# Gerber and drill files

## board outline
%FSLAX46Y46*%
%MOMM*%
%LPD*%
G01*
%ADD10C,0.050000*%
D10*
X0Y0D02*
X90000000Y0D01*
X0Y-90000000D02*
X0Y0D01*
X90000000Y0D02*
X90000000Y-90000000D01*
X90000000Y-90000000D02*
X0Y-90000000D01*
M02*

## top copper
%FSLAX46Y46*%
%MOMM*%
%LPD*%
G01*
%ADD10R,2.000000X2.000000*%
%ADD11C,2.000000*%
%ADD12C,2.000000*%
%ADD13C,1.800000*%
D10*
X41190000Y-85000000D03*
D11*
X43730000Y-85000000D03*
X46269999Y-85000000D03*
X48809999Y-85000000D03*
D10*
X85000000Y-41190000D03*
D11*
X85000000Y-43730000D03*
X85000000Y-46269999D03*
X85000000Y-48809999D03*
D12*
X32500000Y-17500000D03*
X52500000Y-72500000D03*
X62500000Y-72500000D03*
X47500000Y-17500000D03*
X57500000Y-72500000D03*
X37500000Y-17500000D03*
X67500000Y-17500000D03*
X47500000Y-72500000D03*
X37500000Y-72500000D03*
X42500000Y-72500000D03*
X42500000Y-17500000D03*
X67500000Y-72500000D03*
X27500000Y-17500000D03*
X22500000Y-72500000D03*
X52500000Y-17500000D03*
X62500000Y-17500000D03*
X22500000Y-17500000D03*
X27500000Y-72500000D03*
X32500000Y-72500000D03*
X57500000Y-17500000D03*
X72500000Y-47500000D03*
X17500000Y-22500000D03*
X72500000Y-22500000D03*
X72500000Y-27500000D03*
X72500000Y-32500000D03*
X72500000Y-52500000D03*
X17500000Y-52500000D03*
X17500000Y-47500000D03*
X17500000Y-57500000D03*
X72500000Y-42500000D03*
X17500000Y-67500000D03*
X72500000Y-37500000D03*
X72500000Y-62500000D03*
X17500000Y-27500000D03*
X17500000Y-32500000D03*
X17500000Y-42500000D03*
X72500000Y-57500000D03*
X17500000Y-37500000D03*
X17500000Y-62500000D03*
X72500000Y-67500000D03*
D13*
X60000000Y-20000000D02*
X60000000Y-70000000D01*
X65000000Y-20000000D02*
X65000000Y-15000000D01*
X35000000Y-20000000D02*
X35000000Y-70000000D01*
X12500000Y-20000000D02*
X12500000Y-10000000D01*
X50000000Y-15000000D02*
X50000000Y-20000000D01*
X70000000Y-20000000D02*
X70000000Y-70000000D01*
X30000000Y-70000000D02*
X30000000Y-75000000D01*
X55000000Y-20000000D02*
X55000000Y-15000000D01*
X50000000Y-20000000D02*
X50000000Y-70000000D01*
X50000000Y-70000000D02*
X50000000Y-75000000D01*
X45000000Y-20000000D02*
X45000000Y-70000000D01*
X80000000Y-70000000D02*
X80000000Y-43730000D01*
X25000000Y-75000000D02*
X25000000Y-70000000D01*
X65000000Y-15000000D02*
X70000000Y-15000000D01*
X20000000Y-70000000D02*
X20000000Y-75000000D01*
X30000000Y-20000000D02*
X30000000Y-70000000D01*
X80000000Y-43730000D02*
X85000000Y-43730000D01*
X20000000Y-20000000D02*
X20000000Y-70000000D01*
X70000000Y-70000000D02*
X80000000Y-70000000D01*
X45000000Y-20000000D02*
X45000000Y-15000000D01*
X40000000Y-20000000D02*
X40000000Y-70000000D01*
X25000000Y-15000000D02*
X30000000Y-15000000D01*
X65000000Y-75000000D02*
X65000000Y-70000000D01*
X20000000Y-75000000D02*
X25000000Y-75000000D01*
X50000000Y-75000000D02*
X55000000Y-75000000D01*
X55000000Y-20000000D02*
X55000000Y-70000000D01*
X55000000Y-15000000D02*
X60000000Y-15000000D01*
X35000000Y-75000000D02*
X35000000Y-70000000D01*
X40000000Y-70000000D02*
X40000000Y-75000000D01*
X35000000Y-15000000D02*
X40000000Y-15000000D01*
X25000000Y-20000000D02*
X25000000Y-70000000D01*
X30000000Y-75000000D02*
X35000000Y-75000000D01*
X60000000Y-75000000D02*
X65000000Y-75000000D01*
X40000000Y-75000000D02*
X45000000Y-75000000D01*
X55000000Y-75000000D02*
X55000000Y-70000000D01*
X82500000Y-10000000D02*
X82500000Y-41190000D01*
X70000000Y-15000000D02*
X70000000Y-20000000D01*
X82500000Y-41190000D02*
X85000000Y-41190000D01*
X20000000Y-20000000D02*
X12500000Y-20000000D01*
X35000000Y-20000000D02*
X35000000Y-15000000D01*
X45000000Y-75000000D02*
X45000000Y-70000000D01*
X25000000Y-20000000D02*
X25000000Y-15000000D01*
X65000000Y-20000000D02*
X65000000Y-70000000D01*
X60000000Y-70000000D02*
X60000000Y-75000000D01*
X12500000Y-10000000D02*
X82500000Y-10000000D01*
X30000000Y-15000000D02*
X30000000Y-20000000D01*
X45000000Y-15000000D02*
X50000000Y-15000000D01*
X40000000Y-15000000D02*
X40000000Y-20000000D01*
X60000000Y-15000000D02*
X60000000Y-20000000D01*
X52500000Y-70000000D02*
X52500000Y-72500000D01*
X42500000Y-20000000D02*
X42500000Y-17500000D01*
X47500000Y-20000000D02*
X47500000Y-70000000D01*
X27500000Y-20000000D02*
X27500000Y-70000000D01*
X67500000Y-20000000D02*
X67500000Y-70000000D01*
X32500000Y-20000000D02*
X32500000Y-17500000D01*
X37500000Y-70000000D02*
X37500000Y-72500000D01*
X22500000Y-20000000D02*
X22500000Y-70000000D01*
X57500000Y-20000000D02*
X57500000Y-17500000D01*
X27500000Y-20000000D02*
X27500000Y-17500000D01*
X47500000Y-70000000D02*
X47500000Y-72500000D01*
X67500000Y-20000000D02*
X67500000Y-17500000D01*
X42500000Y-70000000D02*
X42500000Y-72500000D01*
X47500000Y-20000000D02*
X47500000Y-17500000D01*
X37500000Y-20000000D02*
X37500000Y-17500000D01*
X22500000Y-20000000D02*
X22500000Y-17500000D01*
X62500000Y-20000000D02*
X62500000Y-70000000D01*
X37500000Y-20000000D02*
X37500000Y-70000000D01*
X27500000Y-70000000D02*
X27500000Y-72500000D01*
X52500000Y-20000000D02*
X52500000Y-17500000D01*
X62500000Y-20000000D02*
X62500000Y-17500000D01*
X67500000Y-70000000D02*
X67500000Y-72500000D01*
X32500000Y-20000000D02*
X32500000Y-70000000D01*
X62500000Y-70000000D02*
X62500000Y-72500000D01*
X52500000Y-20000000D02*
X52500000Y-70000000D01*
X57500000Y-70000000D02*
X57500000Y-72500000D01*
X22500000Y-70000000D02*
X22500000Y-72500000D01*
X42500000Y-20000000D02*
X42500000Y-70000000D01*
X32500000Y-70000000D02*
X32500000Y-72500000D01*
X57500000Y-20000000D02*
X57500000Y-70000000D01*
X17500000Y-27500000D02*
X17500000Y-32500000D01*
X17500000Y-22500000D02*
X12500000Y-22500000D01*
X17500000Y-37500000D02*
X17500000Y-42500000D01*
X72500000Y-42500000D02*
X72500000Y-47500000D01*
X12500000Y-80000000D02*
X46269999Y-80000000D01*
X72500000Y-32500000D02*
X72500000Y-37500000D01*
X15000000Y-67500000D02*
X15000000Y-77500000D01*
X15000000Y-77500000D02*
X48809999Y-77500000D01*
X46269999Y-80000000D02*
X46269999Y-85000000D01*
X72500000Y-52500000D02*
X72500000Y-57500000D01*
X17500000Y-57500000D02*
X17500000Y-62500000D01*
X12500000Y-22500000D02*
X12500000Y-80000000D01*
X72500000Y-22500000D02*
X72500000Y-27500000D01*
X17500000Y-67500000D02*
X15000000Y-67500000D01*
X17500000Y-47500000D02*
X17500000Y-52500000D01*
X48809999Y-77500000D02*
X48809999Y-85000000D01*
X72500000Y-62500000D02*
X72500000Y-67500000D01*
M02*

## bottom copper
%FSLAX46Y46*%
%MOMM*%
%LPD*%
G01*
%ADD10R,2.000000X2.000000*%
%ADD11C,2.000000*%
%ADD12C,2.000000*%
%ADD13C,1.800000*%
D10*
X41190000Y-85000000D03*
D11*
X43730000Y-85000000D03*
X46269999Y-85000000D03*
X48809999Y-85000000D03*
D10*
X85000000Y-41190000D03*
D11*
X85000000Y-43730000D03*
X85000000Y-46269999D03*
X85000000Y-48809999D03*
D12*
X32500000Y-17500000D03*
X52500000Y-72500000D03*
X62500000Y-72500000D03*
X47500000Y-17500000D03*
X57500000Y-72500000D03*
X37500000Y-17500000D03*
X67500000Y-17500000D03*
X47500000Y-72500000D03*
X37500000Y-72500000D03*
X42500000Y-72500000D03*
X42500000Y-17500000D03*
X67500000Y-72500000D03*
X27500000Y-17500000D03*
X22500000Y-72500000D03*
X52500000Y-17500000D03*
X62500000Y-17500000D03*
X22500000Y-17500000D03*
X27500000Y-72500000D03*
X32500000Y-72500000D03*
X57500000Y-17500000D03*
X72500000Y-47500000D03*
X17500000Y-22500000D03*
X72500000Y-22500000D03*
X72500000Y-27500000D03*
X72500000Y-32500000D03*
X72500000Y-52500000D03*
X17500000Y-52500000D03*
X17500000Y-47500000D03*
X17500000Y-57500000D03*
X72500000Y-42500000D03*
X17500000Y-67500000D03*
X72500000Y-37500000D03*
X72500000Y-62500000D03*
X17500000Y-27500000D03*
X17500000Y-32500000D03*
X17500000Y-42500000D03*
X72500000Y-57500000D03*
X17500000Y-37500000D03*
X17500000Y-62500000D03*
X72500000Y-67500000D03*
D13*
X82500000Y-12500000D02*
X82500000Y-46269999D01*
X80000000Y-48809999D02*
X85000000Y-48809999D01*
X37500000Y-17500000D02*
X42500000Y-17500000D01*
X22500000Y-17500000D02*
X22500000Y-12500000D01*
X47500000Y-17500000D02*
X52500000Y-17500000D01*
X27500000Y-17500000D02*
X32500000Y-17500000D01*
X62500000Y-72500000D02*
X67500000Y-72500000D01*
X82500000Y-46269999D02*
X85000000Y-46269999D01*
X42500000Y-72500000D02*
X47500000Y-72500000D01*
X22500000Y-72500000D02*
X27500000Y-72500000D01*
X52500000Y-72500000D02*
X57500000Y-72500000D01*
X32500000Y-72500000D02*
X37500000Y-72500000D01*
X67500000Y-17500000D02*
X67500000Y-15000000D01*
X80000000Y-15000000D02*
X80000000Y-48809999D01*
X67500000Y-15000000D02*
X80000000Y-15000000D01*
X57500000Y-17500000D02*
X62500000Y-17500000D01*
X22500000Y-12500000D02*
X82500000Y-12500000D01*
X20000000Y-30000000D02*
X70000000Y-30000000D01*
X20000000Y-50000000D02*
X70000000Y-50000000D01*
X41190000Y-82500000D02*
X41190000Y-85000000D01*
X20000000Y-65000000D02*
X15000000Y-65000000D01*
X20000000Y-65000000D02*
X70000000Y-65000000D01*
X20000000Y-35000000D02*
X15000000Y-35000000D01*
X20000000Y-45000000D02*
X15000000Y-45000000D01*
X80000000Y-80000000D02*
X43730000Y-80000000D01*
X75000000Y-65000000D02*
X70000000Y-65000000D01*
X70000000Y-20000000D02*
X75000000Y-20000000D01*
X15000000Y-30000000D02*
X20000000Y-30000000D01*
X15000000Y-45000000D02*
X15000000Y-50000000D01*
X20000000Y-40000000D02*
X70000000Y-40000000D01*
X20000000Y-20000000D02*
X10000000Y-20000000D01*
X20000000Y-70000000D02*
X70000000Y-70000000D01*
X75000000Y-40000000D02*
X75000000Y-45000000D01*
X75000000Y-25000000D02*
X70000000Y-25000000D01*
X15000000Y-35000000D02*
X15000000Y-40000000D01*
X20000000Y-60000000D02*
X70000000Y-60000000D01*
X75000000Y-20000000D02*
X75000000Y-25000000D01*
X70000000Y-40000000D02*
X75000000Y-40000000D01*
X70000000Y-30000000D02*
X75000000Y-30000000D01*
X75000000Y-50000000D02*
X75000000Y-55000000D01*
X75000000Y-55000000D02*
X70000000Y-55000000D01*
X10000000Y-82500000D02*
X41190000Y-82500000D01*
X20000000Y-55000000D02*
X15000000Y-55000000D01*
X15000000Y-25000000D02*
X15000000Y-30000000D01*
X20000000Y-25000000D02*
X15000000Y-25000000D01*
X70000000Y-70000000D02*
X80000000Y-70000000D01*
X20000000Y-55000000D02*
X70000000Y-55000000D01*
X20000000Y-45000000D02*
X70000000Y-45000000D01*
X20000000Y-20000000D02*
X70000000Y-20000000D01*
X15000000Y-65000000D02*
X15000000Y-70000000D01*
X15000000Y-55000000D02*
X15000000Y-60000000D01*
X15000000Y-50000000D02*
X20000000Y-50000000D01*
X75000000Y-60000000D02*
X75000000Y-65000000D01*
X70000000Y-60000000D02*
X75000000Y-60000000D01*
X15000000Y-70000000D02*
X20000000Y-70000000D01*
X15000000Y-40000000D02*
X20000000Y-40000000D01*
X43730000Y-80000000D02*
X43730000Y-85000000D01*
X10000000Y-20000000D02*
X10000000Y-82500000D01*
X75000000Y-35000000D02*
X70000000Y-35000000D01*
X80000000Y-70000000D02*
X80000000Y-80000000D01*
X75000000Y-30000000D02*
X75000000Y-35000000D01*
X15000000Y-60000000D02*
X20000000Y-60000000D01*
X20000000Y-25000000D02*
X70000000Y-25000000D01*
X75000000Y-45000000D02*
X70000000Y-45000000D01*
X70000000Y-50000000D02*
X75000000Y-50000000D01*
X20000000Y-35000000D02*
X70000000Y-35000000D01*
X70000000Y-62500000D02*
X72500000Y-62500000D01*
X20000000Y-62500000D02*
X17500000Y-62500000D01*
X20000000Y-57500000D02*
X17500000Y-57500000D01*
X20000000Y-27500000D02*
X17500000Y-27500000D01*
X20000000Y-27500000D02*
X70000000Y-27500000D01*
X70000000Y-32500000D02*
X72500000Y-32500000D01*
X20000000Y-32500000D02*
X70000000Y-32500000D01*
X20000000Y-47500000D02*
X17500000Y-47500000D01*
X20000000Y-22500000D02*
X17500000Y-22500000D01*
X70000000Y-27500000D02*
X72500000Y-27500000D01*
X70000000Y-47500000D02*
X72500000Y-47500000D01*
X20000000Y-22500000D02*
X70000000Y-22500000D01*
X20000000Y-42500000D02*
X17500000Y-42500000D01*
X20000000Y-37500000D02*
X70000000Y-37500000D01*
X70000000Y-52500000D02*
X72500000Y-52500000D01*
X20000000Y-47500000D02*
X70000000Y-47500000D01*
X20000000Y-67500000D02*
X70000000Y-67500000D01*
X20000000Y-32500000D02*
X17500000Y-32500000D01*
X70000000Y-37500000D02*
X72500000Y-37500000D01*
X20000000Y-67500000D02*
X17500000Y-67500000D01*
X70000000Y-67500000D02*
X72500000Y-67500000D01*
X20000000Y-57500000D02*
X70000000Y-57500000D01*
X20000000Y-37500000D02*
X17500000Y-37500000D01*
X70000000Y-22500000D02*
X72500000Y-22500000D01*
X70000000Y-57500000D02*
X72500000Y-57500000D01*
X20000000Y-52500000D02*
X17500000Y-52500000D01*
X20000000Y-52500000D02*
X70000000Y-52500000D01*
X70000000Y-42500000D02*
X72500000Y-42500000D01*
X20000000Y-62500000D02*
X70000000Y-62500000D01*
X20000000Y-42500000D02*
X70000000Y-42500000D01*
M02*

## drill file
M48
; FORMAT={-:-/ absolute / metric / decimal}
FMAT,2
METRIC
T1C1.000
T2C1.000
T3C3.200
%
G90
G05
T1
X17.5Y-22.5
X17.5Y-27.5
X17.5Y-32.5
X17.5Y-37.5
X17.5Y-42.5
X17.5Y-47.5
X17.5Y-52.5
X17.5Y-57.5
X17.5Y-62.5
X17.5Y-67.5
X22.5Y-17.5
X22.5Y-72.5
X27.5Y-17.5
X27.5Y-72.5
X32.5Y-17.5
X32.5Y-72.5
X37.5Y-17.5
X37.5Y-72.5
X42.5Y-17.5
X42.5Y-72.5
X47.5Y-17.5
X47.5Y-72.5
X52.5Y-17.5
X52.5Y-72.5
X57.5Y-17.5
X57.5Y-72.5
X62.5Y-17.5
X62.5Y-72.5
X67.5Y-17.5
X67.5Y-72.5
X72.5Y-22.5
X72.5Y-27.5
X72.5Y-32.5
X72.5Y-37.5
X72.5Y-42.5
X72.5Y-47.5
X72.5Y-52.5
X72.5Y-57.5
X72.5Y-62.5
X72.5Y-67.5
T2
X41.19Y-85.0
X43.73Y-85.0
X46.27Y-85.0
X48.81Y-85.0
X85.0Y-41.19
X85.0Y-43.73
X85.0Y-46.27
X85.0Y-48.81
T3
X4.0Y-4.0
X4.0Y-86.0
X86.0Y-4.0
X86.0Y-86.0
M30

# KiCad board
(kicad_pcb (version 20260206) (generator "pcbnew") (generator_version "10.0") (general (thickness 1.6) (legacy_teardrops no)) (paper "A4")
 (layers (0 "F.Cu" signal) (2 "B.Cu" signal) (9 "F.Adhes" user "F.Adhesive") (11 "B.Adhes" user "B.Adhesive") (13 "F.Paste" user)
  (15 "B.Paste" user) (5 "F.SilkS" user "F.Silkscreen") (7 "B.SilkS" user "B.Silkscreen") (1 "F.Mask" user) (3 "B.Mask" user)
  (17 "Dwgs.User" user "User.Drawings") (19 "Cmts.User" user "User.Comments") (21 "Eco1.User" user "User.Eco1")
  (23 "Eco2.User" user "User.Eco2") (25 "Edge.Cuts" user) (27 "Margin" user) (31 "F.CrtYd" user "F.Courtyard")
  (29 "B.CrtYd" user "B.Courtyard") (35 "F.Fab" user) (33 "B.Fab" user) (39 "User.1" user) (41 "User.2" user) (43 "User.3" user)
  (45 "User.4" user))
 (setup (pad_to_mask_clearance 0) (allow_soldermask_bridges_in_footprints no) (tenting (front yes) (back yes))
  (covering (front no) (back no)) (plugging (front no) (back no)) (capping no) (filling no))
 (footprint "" (layer "F.Cu") (at 86 86)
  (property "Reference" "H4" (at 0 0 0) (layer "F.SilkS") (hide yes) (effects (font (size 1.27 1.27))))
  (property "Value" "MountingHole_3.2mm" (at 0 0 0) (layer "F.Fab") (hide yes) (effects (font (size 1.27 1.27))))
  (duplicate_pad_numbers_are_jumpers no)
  (pad "" np_thru_hole circle (at 0 0) (size 3.2 3.2) (drill 3.2) (layers "*.Cu" "*.Mask")))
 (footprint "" (layer "F.Cu") (at 45 85)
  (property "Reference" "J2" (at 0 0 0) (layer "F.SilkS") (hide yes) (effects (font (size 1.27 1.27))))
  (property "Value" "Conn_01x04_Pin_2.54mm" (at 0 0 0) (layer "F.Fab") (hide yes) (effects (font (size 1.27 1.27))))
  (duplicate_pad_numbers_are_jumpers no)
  (pad "1" thru_hole rect (at -3.81 0) (size 2 2) (drill 1) (layers "*.Cu" "*.Mask") (remove_unused_layers no) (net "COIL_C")
   (thermal_bridge_angle 45))
  (pad "2" thru_hole circle (at -1.27 0) (size 2 2) (drill 1) (layers "*.Cu" "*.Mask") (remove_unused_layers no) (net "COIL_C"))
  (pad "3" thru_hole circle (at 1.269999 0) (size 2 2) (drill 1) (layers "*.Cu" "*.Mask") (remove_unused_layers no) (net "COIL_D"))
  (pad "4" thru_hole circle (at 3.809999 0) (size 2 2) (drill 1) (layers "*.Cu" "*.Mask") (remove_unused_layers no) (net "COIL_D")))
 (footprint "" (layer "F.Cu") (at 86 4)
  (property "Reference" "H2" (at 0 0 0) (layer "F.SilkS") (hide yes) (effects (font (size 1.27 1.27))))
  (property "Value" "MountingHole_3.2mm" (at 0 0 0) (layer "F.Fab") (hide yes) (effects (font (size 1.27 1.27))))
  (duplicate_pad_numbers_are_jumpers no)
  (pad "" np_thru_hole circle (at 0 0) (size 3.2 3.2) (drill 3.2) (layers "*.Cu" "*.Mask")))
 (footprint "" (layer "F.Cu") (at 4 86)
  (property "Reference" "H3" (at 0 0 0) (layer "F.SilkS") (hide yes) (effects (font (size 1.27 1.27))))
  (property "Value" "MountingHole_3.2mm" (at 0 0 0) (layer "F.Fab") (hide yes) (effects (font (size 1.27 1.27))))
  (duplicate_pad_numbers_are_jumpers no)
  (pad "" np_thru_hole circle (at 0 0) (size 3.2 3.2) (drill 3.2) (layers "*.Cu" "*.Mask")))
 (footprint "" (layer "F.Cu") (at 4 4)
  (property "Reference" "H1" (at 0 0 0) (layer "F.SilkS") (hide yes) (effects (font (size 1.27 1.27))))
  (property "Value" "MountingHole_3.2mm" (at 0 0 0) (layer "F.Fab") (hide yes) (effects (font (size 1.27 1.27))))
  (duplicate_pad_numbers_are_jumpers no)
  (pad "" np_thru_hole circle (at 0 0) (size 3.2 3.2) (drill 3.2) (layers "*.Cu" "*.Mask")))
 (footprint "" (layer "F.Cu") (at 85 45)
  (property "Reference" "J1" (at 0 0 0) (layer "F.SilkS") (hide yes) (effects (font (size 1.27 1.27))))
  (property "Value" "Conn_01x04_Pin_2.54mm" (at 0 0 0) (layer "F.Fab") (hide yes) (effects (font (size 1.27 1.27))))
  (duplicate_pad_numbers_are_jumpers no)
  (pad "1" thru_hole rect (at 0 -3.81) (size 2 2) (drill 1) (layers "*.Cu" "*.Mask") (remove_unused_layers no) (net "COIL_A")
   (thermal_bridge_angle 45))
  (pad "2" thru_hole circle (at 0 -1.27) (size 2 2) (drill 1) (layers "*.Cu" "*.Mask") (remove_unused_layers no) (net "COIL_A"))
  (pad "3" thru_hole circle (at 0 1.269999) (size 2 2) (drill 1) (layers "*.Cu" "*.Mask") (remove_unused_layers no) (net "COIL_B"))
  (pad "4" thru_hole circle (at 0 3.809999) (size 2 2) (drill 1) (layers "*.Cu" "*.Mask") (remove_unused_layers no) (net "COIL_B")))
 (gr_line (start 0 0) (end 90 0) (stroke (width 0.05) (type default)) (layer "Edge.Cuts"))
 (gr_line (start 0 90) (end 0 0) (stroke (width 0.05) (type default)) (layer "Edge.Cuts"))
 (gr_line (start 90 0) (end 90 90) (stroke (width 0.05) (type default)) (layer "Edge.Cuts"))
 (gr_line (start 90 90) (end 0 90) (stroke (width 0.05) (type default)) (layer "Edge.Cuts"))
 (segment (start 60 20) (end 60 70) (width 1.8) (layer "F.Cu") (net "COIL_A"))
 (segment (start 65 20) (end 65 15) (width 1.8) (layer "F.Cu") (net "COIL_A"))
 (segment (start 35 20) (end 35 70) (width 1.8) (layer "F.Cu") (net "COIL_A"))
 (segment (start 12.5 20) (end 12.5 10) (width 1.8) (layer "F.Cu") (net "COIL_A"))
 (segment (start 50 15) (end 50 20) (width 1.8) (layer "F.Cu") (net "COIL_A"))
 (segment (start 70 20) (end 70 70) (width 1.8) (layer "F.Cu") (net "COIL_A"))
 (segment (start 30 70) (end 30 75) (width 1.8) (layer "F.Cu") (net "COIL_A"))
 (segment (start 55 20) (end 55 15) (width 1.8) (layer "F.Cu") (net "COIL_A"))
 (segment (start 50 20) (end 50 70) (width 1.8) (layer "F.Cu") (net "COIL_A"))
 (segment (start 50 70) (end 50 75) (width 1.8) (layer "F.Cu") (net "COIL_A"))
 (segment (start 45 20) (end 45 70) (width 1.8) (layer "F.Cu") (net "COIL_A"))
 (segment (start 80 70) (end 80 43.73) (width 1.8) (layer "F.Cu") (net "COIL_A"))
 (segment (start 25 75) (end 25 70) (width 1.8) (layer "F.Cu") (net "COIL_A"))
 (segment (start 65 15) (end 70 15) (width 1.8) (layer "F.Cu") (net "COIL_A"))
 (segment (start 20 70) (end 20 75) (width 1.8) (layer "F.Cu") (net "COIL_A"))
 (segment (start 30 20) (end 30 70) (width 1.8) (layer "F.Cu") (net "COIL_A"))
 (segment (start 80 43.73) (end 85 43.73) (width 1.8) (layer "F.Cu") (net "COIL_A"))
 (segment (start 20 20) (end 20 70) (width 1.8) (layer "F.Cu") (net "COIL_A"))
 (segment (start 70 70) (end 80 70) (width 1.8) (layer "F.Cu") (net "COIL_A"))
 (segment (start 45 20) (end 45 15) (width 1.8) (layer "F.Cu") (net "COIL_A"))
 (segment (start 40 20) (end 40 70) (width 1.8) (layer "F.Cu") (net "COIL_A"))
 (segment (start 25 15) (end 30 15) (width 1.8) (layer "F.Cu") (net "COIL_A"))
 (segment (start 65 75) (end 65 70) (width 1.8) (layer "F.Cu") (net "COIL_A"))
 (segment (start 20 75) (end 25 75) (width 1.8) (layer "F.Cu") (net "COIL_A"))
 (segment (start 50 75) (end 55 75) (width 1.8) (layer "F.Cu") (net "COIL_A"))
 (segment (start 55 20) (end 55 70) (width 1.8) (layer "F.Cu") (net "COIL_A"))
 (segment (start 55 15) (end 60 15) (width 1.8) (layer "F.Cu") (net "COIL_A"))
 (segment (start 35 75) (end 35 70) (width 1.8) (layer "F.Cu") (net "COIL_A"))
 (segment (start 40 70) (end 40 75) (width 1.8) (layer "F.Cu") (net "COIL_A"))
 (segment (start 35 15) (end 40 15) (width 1.8) (layer "F.Cu") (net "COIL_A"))
 (segment (start 25 20) (end 25 70) (width 1.8) (layer "F.Cu") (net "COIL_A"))
 (segment (start 30 75) (end 35 75) (width 1.8) (layer "F.Cu") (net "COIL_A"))
 (segment (start 60 75) (end 65 75) (width 1.8) (layer "F.Cu") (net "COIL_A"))
 (segment (start 40 75) (end 45 75) (width 1.8) (layer "F.Cu") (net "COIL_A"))
 (segment (start 55 75) (end 55 70) (width 1.8) (layer "F.Cu") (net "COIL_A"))
 (segment (start 82.5 10) (end 82.5 41.19) (width 1.8) (layer "F.Cu") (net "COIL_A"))
 (segment (start 70 15) (end 70 20) (width 1.8) (layer "F.Cu") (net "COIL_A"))
 (segment (start 82.5 41.19) (end 85 41.19) (width 1.8) (layer "F.Cu") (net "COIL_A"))
 (segment (start 20 20) (end 12.5 20) (width 1.8) (layer "F.Cu") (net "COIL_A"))
 (segment (start 35 20) (end 35 15) (width 1.8) (layer "F.Cu") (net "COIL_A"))
 (segment (start 45 75) (end 45 70) (width 1.8) (layer "F.Cu") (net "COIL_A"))
 (segment (start 25 20) (end 25 15) (width 1.8) (layer "F.Cu") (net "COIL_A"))
 (segment (start 65 20) (end 65 70) (width 1.8) (layer "F.Cu") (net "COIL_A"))
 (segment (start 60 70) (end 60 75) (width 1.8) (layer "F.Cu") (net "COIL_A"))
 (segment (start 12.5 10) (end 82.5 10) (width 1.8) (layer "F.Cu") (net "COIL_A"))
 (segment (start 30 15) (end 30 20) (width 1.8) (layer "F.Cu") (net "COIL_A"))
 (segment (start 45 15) (end 50 15) (width 1.8) (layer "F.Cu") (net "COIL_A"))
 (segment (start 40 15) (end 40 20) (width 1.8) (layer "F.Cu") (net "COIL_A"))
 (segment (start 60 15) (end 60 20) (width 1.8) (layer "F.Cu") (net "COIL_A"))
 (segment (start 52.5 70) (end 52.5 72.5) (width 1.8) (layer "F.Cu") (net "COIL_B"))
 (segment (start 42.5 20) (end 42.5 17.5) (width 1.8) (layer "F.Cu") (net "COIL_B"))
 (segment (start 47.5 20) (end 47.5 70) (width 1.8) (layer "F.Cu") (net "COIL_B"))
 (segment (start 27.5 20) (end 27.5 70) (width 1.8) (layer "F.Cu") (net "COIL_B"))
 (segment (start 67.5 20) (end 67.5 70) (width 1.8) (layer "F.Cu") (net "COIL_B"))
 (segment (start 32.5 20) (end 32.5 17.5) (width 1.8) (layer "F.Cu") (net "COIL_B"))
 (segment (start 37.5 70) (end 37.5 72.5) (width 1.8) (layer "F.Cu") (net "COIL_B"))
 (segment (start 22.5 20) (end 22.5 70) (width 1.8) (layer "F.Cu") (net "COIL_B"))
 (segment (start 57.5 20) (end 57.5 17.5) (width 1.8) (layer "F.Cu") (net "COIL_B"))
 (segment (start 27.5 20) (end 27.5 17.5) (width 1.8) (layer "F.Cu") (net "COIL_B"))
 (segment (start 47.5 70) (end 47.5 72.5) (width 1.8) (layer "F.Cu") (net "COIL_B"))
 (segment (start 67.5 20) (end 67.5 17.5) (width 1.8) (layer "F.Cu") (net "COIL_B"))
 (segment (start 42.5 70) (end 42.5 72.5) (width 1.8) (layer "F.Cu") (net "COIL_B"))
 (segment (start 47.5 20) (end 47.5 17.5) (width 1.8) (layer "F.Cu") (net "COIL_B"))
 (segment (start 37.5 20) (end 37.5 17.5) (width 1.8) (layer "F.Cu") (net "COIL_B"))
 (segment (start 22.5 20) (end 22.5 17.5) (width 1.8) (layer "F.Cu") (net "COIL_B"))
 (segment (start 62.5 20) (end 62.5 70) (width 1.8) (layer "F.Cu") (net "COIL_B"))
 (segment (start 37.5 20) (end 37.5 70) (width 1.8) (layer "F.Cu") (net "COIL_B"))
 (segment (start 27.5 70) (end 27.5 72.5) (width 1.8) (layer "F.Cu") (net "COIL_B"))
 (segment (start 52.5 20) (end 52.5 17.5) (width 1.8) (layer "F.Cu") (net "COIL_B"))
 (segment (start 62.5 20) (end 62.5 17.5) (width 1.8) (layer "F.Cu") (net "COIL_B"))
 (segment (start 67.5 70) (end 67.5 72.5) (width 1.8) (layer "F.Cu") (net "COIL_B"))
 (segment (start 32.5 20) (end 32.5 70) (width 1.8) (layer "F.Cu") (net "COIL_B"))
 (segment (start 62.5 70) (end 62.5 72.5) (width 1.8) (layer "F.Cu") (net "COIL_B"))
 (segment (start 52.5 20) (end 52.5 70) (width 1.8) (layer "F.Cu") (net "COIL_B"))
 (segment (start 57.5 70) (end 57.5 72.5) (width 1.8) (layer "F.Cu") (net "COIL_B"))
 (segment (start 22.5 70) (end 22.5 72.5) (width 1.8) (layer "F.Cu") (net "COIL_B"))
 (segment (start 42.5 20) (end 42.5 70) (width 1.8) (layer "F.Cu") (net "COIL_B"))
 (segment (start 32.5 70) (end 32.5 72.5) (width 1.8) (layer "F.Cu") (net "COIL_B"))
 (segment (start 57.5 20) (end 57.5 70) (width 1.8) (layer "F.Cu") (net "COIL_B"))
 (via (at 32.5 17.5) (size 2) (drill 1) (layers "F.Cu" "B.Cu") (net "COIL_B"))
 (via (at 52.5 72.5) (size 2) (drill 1) (layers "F.Cu" "B.Cu") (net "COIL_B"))
 (via (at 62.5 72.5) (size 2) (drill 1) (layers "F.Cu" "B.Cu") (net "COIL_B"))
 (via (at 47.5 17.5) (size 2) (drill 1) (layers "F.Cu" "B.Cu") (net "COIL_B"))
 (via (at 57.5 72.5) (size 2) (drill 1) (layers "F.Cu" "B.Cu") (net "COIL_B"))
 (via (at 37.5 17.5) (size 2) (drill 1) (layers "F.Cu" "B.Cu") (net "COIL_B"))
 (via (at 67.5 17.5) (size 2) (drill 1) (layers "F.Cu" "B.Cu") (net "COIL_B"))
 (via (at 47.5 72.5) (size 2) (drill 1) (layers "F.Cu" "B.Cu") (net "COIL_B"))
 (via (at 37.5 72.5) (size 2) (drill 1) (layers "F.Cu" "B.Cu") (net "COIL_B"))
 (via (at 42.5 72.5) (size 2) (drill 1) (layers "F.Cu" "B.Cu") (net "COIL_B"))
 (via (at 42.5 17.5) (size 2) (drill 1) (layers "F.Cu" "B.Cu") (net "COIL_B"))
 (via (at 67.5 72.5) (size 2) (drill 1) (layers "F.Cu" "B.Cu") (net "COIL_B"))
 (via (at 27.5 17.5) (size 2) (drill 1) (layers "F.Cu" "B.Cu") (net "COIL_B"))
 (via (at 22.5 72.5) (size 2) (drill 1) (layers "F.Cu" "B.Cu") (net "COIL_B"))
 (via (at 52.5 17.5) (size 2) (drill 1) (layers "F.Cu" "B.Cu") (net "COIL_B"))
 (via (at 62.5 17.5) (size 2) (drill 1) (layers "F.Cu" "B.Cu") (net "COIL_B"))
 (via (at 22.5 17.5) (size 2) (drill 1) (layers "F.Cu" "B.Cu") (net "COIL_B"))
 (via (at 27.5 72.5) (size 2) (drill 1) (layers "F.Cu" "B.Cu") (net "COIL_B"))
 (via (at 32.5 72.5) (size 2) (drill 1) (layers "F.Cu" "B.Cu") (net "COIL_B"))
 (via (at 57.5 17.5) (size 2) (drill 1) (layers "F.Cu" "B.Cu") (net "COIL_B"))
 (segment (start 82.5 12.5) (end 82.5 46.269999) (width 1.8) (layer "B.Cu") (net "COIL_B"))
 (segment (start 80 48.809999) (end 85 48.809999) (width 1.8) (layer "B.Cu") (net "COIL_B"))
 (segment (start 37.5 17.5) (end 42.5 17.5) (width 1.8) (layer "B.Cu") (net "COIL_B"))
 (segment (start 22.5 17.5) (end 22.5 12.5) (width 1.8) (layer "B.Cu") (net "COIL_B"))
 (segment (start 47.5 17.5) (end 52.5 17.5) (width 1.8) (layer "B.Cu") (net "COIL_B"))
 (segment (start 27.5 17.5) (end 32.5 17.5) (width 1.8) (layer "B.Cu") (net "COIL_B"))
 (segment (start 62.5 72.5) (end 67.5 72.5) (width 1.8) (layer "B.Cu") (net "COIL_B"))
 (segment (start 82.5 46.269999) (end 85 46.269999) (width 1.8) (layer "B.Cu") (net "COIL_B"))
 (segment (start 42.5 72.5) (end 47.5 72.5) (width 1.8) (layer "B.Cu") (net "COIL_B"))
 (segment (start 22.5 72.5) (end 27.5 72.5) (width 1.8) (layer "B.Cu") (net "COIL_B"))
 (segment (start 52.5 72.5) (end 57.5 72.5) (width 1.8) (layer "B.Cu") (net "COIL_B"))
 (segment (start 32.5 72.5) (end 37.5 72.5) (width 1.8) (layer "B.Cu") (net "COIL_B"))
 (segment (start 67.5 17.5) (end 67.5 15) (width 1.8) (layer "B.Cu") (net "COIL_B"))
 (segment (start 80 15) (end 80 48.809999) (width 1.8) (layer "B.Cu") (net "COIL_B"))
 (segment (start 67.5 15) (end 80 15) (width 1.8) (layer "B.Cu") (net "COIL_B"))
 (segment (start 57.5 17.5) (end 62.5 17.5) (width 1.8) (layer "B.Cu") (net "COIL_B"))
 (segment (start 22.5 12.5) (end 82.5 12.5) (width 1.8) (layer "B.Cu") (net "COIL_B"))
 (segment (start 20 30) (end 70 30) (width 1.8) (layer "B.Cu") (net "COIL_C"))
 (segment (start 20 50) (end 70 50) (width 1.8) (layer "B.Cu") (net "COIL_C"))
 (segment (start 41.19 82.5) (end 41.19 85) (width 1.8) (layer "B.Cu") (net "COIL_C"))
 (segment (start 20 65) (end 15 65) (width 1.8) (layer "B.Cu") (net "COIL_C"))
 (segment (start 20 65) (end 70 65) (width 1.8) (layer "B.Cu") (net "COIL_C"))
 (segment (start 20 35) (end 15 35) (width 1.8) (layer "B.Cu") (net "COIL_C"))
 (segment (start 20 45) (end 15 45) (width 1.8) (layer "B.Cu") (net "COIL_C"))
 (segment (start 80 80) (end 43.73 80) (width 1.8) (layer "B.Cu") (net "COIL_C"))
 (segment (start 75 65) (end 70 65) (width 1.8) (layer "B.Cu") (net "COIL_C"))
 (segment (start 70 20) (end 75 20) (width 1.8) (layer "B.Cu") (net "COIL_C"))
 (segment (start 15 30) (end 20 30) (width 1.8) (layer "B.Cu") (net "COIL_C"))
 (segment (start 15 45) (end 15 50) (width 1.8) (layer "B.Cu") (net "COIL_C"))
 (segment (start 20 40) (end 70 40) (width 1.8) (layer "B.Cu") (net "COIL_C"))
 (segment (start 20 20) (end 10 20) (width 1.8) (layer "B.Cu") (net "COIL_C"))
 (segment (start 20 70) (end 70 70) (width 1.8) (layer "B.Cu") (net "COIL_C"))
 (segment (start 75 40) (end 75 45) (width 1.8) (layer "B.Cu") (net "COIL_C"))
 (segment (start 75 25) (end 70 25) (width 1.8) (layer "B.Cu") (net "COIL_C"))
 (segment (start 15 35) (end 15 40) (width 1.8) (layer "B.Cu") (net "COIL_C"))
 (segment (start 20 60) (end 70 60) (width 1.8) (layer "B.Cu") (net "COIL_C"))
 (segment (start 75 20) (end 75 25) (width 1.8) (layer "B.Cu") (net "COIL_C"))
 (segment (start 70 40) (end 75 40) (width 1.8) (layer "B.Cu") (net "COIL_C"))
 (segment (start 70 30) (end 75 30) (width 1.8) (layer "B.Cu") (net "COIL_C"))
 (segment (start 75 50) (end 75 55) (width 1.8) (layer "B.Cu") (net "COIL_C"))
 (segment (start 75 55) (end 70 55) (width 1.8) (layer "B.Cu") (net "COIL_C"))
 (segment (start 10 82.5) (end 41.19 82.5) (width 1.8) (layer "B.Cu") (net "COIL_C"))
 (segment (start 20 55) (end 15 55) (width 1.8) (layer "B.Cu") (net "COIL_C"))
 (segment (start 15 25) (end 15 30) (width 1.8) (layer "B.Cu") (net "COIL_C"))
 (segment (start 20 25) (end 15 25) (width 1.8) (layer "B.Cu") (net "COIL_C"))
 (segment (start 70 70) (end 80 70) (width 1.8) (layer "B.Cu") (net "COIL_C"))
 (segment (start 20 55) (end 70 55) (width 1.8) (layer "B.Cu") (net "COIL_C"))
 (segment (start 20 45) (end 70 45) (width 1.8) (layer "B.Cu") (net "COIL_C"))
 (segment (start 20 20) (end 70 20) (width 1.8) (layer "B.Cu") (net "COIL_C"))
 (segment (start 15 65) (end 15 70) (width 1.8) (layer "B.Cu") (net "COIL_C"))
 (segment (start 15 55) (end 15 60) (width 1.8) (layer "B.Cu") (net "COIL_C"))
 (segment (start 15 50) (end 20 50) (width 1.8) (layer "B.Cu") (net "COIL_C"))
 (segment (start 75 60) (end 75 65) (width 1.8) (layer "B.Cu") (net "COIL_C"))
 (segment (start 70 60) (end 75 60) (width 1.8) (layer "B.Cu") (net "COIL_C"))
 (segment (start 15 70) (end 20 70) (width 1.8) (layer "B.Cu") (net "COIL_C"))
 (segment (start 15 40) (end 20 40) (width 1.8) (layer "B.Cu") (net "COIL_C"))
 (segment (start 43.73 80) (end 43.73 85) (width 1.8) (layer "B.Cu") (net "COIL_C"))
 (segment (start 10 20) (end 10 82.5) (width 1.8) (layer "B.Cu") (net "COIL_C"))
 (segment (start 75 35) (end 70 35) (width 1.8) (layer "B.Cu") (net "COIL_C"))
 (segment (start 80 70) (end 80 80) (width 1.8) (layer "B.Cu") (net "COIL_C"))
 (segment (start 75 30) (end 75 35) (width 1.8) (layer "B.Cu") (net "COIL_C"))
 (segment (start 15 60) (end 20 60) (width 1.8) (layer "B.Cu") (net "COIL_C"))
 (segment (start 20 25) (end 70 25) (width 1.8) (layer "B.Cu") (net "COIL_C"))
 (segment (start 75 45) (end 70 45) (width 1.8) (layer "B.Cu") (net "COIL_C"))
 (segment (start 70 50) (end 75 50) (width 1.8) (layer "B.Cu") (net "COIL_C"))
 (segment (start 20 35) (end 70 35) (width 1.8) (layer "B.Cu") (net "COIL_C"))
 (segment (start 17.5 27.5) (end 17.5 32.5) (width 1.8) (layer "F.Cu") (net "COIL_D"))
 (segment (start 17.5 22.5) (end 12.5 22.5) (width 1.8) (layer "F.Cu") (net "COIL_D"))
 (segment (start 17.5 37.5) (end 17.5 42.5) (width 1.8) (layer "F.Cu") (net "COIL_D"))
 (segment (start 72.5 42.5) (end 72.5 47.5) (width 1.8) (layer "F.Cu") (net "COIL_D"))
 (segment (start 12.5 80) (end 46.269999 80) (width 1.8) (layer "F.Cu") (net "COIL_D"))
 (segment (start 72.5 32.5) (end 72.5 37.5) (width 1.8) (layer "F.Cu") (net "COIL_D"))
 (segment (start 15 67.5) (end 15 77.5) (width 1.8) (layer "F.Cu") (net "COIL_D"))
 (segment (start 15 77.5) (end 48.809999 77.5) (width 1.8) (layer "F.Cu") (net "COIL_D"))
 (segment (start 46.269999 80) (end 46.269999 85) (width 1.8) (layer "F.Cu") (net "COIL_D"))
 (segment (start 72.5 52.5) (end 72.5 57.5) (width 1.8) (layer "F.Cu") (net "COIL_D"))
 (segment (start 17.5 57.5) (end 17.5 62.5) (width 1.8) (layer "F.Cu") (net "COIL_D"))
 (segment (start 12.5 22.5) (end 12.5 80) (width 1.8) (layer "F.Cu") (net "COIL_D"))
 (segment (start 72.5 22.5) (end 72.5 27.5) (width 1.8) (layer "F.Cu") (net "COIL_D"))
 (segment (start 17.5 67.5) (end 15 67.5) (width 1.8) (layer "F.Cu") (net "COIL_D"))
 (segment (start 17.5 47.5) (end 17.5 52.5) (width 1.8) (layer "F.Cu") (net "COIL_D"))
 (segment (start 48.809999 77.5) (end 48.809999 85) (width 1.8) (layer "F.Cu") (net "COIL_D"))
 (segment (start 72.5 62.5) (end 72.5 67.5) (width 1.8) (layer "F.Cu") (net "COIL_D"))
 (via (at 72.5 47.5) (size 2) (drill 1) (layers "F.Cu" "B.Cu") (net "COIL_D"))
 (via (at 17.5 22.5) (size 2) (drill 1) (layers "F.Cu" "B.Cu") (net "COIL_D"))
 (via (at 72.5 22.5) (size 2) (drill 1) (layers "F.Cu" "B.Cu") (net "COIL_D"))
 (via (at 72.5 27.5) (size 2) (drill 1) (layers "F.Cu" "B.Cu") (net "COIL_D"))
 (via (at 72.5 32.5) (size 2) (drill 1) (layers "F.Cu" "B.Cu") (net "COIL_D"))
 (via (at 72.5 52.5) (size 2) (drill 1) (layers "F.Cu" "B.Cu") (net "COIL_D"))
 (via (at 17.5 52.5) (size 2) (drill 1) (layers "F.Cu" "B.Cu") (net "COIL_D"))
 (via (at 17.5 47.5) (size 2) (drill 1) (layers "F.Cu" "B.Cu") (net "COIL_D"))
 (via (at 17.5 57.5) (size 2) (drill 1) (layers "F.Cu" "B.Cu") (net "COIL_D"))
 (via (at 72.5 42.5) (size 2) (drill 1) (layers "F.Cu" "B.Cu") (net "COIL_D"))
 (via (at 17.5 67.5) (size 2) (drill 1) (layers "F.Cu" "B.Cu") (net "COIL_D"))
 (via (at 72.5 37.5) (size 2) (drill 1) (layers "F.Cu" "B.Cu") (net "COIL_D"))
 (via (at 72.5 62.5) (size 2) (drill 1) (layers "F.Cu" "B.Cu") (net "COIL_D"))
 (via (at 17.5 27.5) (size 2) (drill 1) (layers "F.Cu" "B.Cu") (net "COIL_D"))
 (via (at 17.5 32.5) (size 2) (drill 1) (layers "F.Cu" "B.Cu") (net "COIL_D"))
 (via (at 17.5 42.5) (size 2) (drill 1) (layers "F.Cu" "B.Cu") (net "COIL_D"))
 (via (at 72.5 57.5) (size 2) (drill 1) (layers "F.Cu" "B.Cu") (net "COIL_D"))
 (via (at 17.5 37.5) (size 2) (drill 1) (layers "F.Cu" "B.Cu") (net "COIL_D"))
 (via (at 17.5 62.5) (size 2) (drill 1) (layers "F.Cu" "B.Cu") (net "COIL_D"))
 (via (at 72.5 67.5) (size 2) (drill 1) (layers "F.Cu" "B.Cu") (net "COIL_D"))
 (segment (start 70 62.5) (end 72.5 62.5) (width 1.8) (layer "B.Cu") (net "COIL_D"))
 (segment (start 20 62.5) (end 17.5 62.5) (width 1.8) (layer "B.Cu") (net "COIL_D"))
 (segment (start 20 57.5) (end 17.5 57.5) (width 1.8) (layer "B.Cu") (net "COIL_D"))
 (segment (start 20 27.5) (end 17.5 27.5) (width 1.8) (layer "B.Cu") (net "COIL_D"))
 (segment (start 20 27.5) (end 70 27.5) (width 1.8) (layer "B.Cu") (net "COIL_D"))
 (segment (start 70 32.5) (end 72.5 32.5) (width 1.8) (layer "B.Cu") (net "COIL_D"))
 (segment (start 20 32.5) (end 70 32.5) (width 1.8) (layer "B.Cu") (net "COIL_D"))
 (segment (start 20 47.5) (end 17.5 47.5) (width 1.8) (layer "B.Cu") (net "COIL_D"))
 (segment (start 20 22.5) (end 17.5 22.5) (width 1.8) (layer "B.Cu") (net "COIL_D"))
 (segment (start 70 27.5) (end 72.5 27.5) (width 1.8) (layer "B.Cu") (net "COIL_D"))
 (segment (start 70 47.5) (end 72.5 47.5) (width 1.8) (layer "B.Cu") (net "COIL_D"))
 (segment (start 20 22.5) (end 70 22.5) (width 1.8) (layer "B.Cu") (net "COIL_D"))
 (segment (start 20 42.5) (end 17.5 42.5) (width 1.8) (layer "B.Cu") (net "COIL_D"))
 (segment (start 20 37.5) (end 70 37.5) (width 1.8) (layer "B.Cu") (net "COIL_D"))
 (segment (start 70 52.5) (end 72.5 52.5) (width 1.8) (layer "B.Cu") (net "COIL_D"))
 (segment (start 20 47.5) (end 70 47.5) (width 1.8) (layer "B.Cu") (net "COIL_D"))
 (segment (start 20 67.5) (end 70 67.5) (width 1.8) (layer "B.Cu") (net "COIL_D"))
 (segment (start 20 32.5) (end 17.5 32.5) (width 1.8) (layer "B.Cu") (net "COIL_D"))
 (segment (start 70 37.5) (end 72.5 37.5) (width 1.8) (layer "B.Cu") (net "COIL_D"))
 (segment (start 20 67.5) (end 17.5 67.5) (width 1.8) (layer "B.Cu") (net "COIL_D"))
 (segment (start 70 67.5) (end 72.5 67.5) (width 1.8) (layer "B.Cu") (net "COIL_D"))
 (segment (start 20 57.5) (end 70 57.5) (width 1.8) (layer "B.Cu") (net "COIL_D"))
 (segment (start 20 37.5) (end 17.5 37.5) (width 1.8) (layer "B.Cu") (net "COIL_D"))
 (segment (start 70 22.5) (end 72.5 22.5) (width 1.8) (layer "B.Cu") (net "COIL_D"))
 (segment (start 70 57.5) (end 72.5 57.5) (width 1.8) (layer "B.Cu") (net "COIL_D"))
 (segment (start 20 52.5) (end 17.5 52.5) (width 1.8) (layer "B.Cu") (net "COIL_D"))
 (segment (start 20 52.5) (end 70 52.5) (width 1.8) (layer "B.Cu") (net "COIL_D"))
 (segment (start 70 42.5) (end 72.5 42.5) (width 1.8) (layer "B.Cu") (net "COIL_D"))
 (segment (start 20 62.5) (end 70 62.5) (width 1.8) (layer "B.Cu") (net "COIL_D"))
 (segment (start 20 42.5) (end 70 42.5) (width 1.8) (layer "B.Cu") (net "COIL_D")))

